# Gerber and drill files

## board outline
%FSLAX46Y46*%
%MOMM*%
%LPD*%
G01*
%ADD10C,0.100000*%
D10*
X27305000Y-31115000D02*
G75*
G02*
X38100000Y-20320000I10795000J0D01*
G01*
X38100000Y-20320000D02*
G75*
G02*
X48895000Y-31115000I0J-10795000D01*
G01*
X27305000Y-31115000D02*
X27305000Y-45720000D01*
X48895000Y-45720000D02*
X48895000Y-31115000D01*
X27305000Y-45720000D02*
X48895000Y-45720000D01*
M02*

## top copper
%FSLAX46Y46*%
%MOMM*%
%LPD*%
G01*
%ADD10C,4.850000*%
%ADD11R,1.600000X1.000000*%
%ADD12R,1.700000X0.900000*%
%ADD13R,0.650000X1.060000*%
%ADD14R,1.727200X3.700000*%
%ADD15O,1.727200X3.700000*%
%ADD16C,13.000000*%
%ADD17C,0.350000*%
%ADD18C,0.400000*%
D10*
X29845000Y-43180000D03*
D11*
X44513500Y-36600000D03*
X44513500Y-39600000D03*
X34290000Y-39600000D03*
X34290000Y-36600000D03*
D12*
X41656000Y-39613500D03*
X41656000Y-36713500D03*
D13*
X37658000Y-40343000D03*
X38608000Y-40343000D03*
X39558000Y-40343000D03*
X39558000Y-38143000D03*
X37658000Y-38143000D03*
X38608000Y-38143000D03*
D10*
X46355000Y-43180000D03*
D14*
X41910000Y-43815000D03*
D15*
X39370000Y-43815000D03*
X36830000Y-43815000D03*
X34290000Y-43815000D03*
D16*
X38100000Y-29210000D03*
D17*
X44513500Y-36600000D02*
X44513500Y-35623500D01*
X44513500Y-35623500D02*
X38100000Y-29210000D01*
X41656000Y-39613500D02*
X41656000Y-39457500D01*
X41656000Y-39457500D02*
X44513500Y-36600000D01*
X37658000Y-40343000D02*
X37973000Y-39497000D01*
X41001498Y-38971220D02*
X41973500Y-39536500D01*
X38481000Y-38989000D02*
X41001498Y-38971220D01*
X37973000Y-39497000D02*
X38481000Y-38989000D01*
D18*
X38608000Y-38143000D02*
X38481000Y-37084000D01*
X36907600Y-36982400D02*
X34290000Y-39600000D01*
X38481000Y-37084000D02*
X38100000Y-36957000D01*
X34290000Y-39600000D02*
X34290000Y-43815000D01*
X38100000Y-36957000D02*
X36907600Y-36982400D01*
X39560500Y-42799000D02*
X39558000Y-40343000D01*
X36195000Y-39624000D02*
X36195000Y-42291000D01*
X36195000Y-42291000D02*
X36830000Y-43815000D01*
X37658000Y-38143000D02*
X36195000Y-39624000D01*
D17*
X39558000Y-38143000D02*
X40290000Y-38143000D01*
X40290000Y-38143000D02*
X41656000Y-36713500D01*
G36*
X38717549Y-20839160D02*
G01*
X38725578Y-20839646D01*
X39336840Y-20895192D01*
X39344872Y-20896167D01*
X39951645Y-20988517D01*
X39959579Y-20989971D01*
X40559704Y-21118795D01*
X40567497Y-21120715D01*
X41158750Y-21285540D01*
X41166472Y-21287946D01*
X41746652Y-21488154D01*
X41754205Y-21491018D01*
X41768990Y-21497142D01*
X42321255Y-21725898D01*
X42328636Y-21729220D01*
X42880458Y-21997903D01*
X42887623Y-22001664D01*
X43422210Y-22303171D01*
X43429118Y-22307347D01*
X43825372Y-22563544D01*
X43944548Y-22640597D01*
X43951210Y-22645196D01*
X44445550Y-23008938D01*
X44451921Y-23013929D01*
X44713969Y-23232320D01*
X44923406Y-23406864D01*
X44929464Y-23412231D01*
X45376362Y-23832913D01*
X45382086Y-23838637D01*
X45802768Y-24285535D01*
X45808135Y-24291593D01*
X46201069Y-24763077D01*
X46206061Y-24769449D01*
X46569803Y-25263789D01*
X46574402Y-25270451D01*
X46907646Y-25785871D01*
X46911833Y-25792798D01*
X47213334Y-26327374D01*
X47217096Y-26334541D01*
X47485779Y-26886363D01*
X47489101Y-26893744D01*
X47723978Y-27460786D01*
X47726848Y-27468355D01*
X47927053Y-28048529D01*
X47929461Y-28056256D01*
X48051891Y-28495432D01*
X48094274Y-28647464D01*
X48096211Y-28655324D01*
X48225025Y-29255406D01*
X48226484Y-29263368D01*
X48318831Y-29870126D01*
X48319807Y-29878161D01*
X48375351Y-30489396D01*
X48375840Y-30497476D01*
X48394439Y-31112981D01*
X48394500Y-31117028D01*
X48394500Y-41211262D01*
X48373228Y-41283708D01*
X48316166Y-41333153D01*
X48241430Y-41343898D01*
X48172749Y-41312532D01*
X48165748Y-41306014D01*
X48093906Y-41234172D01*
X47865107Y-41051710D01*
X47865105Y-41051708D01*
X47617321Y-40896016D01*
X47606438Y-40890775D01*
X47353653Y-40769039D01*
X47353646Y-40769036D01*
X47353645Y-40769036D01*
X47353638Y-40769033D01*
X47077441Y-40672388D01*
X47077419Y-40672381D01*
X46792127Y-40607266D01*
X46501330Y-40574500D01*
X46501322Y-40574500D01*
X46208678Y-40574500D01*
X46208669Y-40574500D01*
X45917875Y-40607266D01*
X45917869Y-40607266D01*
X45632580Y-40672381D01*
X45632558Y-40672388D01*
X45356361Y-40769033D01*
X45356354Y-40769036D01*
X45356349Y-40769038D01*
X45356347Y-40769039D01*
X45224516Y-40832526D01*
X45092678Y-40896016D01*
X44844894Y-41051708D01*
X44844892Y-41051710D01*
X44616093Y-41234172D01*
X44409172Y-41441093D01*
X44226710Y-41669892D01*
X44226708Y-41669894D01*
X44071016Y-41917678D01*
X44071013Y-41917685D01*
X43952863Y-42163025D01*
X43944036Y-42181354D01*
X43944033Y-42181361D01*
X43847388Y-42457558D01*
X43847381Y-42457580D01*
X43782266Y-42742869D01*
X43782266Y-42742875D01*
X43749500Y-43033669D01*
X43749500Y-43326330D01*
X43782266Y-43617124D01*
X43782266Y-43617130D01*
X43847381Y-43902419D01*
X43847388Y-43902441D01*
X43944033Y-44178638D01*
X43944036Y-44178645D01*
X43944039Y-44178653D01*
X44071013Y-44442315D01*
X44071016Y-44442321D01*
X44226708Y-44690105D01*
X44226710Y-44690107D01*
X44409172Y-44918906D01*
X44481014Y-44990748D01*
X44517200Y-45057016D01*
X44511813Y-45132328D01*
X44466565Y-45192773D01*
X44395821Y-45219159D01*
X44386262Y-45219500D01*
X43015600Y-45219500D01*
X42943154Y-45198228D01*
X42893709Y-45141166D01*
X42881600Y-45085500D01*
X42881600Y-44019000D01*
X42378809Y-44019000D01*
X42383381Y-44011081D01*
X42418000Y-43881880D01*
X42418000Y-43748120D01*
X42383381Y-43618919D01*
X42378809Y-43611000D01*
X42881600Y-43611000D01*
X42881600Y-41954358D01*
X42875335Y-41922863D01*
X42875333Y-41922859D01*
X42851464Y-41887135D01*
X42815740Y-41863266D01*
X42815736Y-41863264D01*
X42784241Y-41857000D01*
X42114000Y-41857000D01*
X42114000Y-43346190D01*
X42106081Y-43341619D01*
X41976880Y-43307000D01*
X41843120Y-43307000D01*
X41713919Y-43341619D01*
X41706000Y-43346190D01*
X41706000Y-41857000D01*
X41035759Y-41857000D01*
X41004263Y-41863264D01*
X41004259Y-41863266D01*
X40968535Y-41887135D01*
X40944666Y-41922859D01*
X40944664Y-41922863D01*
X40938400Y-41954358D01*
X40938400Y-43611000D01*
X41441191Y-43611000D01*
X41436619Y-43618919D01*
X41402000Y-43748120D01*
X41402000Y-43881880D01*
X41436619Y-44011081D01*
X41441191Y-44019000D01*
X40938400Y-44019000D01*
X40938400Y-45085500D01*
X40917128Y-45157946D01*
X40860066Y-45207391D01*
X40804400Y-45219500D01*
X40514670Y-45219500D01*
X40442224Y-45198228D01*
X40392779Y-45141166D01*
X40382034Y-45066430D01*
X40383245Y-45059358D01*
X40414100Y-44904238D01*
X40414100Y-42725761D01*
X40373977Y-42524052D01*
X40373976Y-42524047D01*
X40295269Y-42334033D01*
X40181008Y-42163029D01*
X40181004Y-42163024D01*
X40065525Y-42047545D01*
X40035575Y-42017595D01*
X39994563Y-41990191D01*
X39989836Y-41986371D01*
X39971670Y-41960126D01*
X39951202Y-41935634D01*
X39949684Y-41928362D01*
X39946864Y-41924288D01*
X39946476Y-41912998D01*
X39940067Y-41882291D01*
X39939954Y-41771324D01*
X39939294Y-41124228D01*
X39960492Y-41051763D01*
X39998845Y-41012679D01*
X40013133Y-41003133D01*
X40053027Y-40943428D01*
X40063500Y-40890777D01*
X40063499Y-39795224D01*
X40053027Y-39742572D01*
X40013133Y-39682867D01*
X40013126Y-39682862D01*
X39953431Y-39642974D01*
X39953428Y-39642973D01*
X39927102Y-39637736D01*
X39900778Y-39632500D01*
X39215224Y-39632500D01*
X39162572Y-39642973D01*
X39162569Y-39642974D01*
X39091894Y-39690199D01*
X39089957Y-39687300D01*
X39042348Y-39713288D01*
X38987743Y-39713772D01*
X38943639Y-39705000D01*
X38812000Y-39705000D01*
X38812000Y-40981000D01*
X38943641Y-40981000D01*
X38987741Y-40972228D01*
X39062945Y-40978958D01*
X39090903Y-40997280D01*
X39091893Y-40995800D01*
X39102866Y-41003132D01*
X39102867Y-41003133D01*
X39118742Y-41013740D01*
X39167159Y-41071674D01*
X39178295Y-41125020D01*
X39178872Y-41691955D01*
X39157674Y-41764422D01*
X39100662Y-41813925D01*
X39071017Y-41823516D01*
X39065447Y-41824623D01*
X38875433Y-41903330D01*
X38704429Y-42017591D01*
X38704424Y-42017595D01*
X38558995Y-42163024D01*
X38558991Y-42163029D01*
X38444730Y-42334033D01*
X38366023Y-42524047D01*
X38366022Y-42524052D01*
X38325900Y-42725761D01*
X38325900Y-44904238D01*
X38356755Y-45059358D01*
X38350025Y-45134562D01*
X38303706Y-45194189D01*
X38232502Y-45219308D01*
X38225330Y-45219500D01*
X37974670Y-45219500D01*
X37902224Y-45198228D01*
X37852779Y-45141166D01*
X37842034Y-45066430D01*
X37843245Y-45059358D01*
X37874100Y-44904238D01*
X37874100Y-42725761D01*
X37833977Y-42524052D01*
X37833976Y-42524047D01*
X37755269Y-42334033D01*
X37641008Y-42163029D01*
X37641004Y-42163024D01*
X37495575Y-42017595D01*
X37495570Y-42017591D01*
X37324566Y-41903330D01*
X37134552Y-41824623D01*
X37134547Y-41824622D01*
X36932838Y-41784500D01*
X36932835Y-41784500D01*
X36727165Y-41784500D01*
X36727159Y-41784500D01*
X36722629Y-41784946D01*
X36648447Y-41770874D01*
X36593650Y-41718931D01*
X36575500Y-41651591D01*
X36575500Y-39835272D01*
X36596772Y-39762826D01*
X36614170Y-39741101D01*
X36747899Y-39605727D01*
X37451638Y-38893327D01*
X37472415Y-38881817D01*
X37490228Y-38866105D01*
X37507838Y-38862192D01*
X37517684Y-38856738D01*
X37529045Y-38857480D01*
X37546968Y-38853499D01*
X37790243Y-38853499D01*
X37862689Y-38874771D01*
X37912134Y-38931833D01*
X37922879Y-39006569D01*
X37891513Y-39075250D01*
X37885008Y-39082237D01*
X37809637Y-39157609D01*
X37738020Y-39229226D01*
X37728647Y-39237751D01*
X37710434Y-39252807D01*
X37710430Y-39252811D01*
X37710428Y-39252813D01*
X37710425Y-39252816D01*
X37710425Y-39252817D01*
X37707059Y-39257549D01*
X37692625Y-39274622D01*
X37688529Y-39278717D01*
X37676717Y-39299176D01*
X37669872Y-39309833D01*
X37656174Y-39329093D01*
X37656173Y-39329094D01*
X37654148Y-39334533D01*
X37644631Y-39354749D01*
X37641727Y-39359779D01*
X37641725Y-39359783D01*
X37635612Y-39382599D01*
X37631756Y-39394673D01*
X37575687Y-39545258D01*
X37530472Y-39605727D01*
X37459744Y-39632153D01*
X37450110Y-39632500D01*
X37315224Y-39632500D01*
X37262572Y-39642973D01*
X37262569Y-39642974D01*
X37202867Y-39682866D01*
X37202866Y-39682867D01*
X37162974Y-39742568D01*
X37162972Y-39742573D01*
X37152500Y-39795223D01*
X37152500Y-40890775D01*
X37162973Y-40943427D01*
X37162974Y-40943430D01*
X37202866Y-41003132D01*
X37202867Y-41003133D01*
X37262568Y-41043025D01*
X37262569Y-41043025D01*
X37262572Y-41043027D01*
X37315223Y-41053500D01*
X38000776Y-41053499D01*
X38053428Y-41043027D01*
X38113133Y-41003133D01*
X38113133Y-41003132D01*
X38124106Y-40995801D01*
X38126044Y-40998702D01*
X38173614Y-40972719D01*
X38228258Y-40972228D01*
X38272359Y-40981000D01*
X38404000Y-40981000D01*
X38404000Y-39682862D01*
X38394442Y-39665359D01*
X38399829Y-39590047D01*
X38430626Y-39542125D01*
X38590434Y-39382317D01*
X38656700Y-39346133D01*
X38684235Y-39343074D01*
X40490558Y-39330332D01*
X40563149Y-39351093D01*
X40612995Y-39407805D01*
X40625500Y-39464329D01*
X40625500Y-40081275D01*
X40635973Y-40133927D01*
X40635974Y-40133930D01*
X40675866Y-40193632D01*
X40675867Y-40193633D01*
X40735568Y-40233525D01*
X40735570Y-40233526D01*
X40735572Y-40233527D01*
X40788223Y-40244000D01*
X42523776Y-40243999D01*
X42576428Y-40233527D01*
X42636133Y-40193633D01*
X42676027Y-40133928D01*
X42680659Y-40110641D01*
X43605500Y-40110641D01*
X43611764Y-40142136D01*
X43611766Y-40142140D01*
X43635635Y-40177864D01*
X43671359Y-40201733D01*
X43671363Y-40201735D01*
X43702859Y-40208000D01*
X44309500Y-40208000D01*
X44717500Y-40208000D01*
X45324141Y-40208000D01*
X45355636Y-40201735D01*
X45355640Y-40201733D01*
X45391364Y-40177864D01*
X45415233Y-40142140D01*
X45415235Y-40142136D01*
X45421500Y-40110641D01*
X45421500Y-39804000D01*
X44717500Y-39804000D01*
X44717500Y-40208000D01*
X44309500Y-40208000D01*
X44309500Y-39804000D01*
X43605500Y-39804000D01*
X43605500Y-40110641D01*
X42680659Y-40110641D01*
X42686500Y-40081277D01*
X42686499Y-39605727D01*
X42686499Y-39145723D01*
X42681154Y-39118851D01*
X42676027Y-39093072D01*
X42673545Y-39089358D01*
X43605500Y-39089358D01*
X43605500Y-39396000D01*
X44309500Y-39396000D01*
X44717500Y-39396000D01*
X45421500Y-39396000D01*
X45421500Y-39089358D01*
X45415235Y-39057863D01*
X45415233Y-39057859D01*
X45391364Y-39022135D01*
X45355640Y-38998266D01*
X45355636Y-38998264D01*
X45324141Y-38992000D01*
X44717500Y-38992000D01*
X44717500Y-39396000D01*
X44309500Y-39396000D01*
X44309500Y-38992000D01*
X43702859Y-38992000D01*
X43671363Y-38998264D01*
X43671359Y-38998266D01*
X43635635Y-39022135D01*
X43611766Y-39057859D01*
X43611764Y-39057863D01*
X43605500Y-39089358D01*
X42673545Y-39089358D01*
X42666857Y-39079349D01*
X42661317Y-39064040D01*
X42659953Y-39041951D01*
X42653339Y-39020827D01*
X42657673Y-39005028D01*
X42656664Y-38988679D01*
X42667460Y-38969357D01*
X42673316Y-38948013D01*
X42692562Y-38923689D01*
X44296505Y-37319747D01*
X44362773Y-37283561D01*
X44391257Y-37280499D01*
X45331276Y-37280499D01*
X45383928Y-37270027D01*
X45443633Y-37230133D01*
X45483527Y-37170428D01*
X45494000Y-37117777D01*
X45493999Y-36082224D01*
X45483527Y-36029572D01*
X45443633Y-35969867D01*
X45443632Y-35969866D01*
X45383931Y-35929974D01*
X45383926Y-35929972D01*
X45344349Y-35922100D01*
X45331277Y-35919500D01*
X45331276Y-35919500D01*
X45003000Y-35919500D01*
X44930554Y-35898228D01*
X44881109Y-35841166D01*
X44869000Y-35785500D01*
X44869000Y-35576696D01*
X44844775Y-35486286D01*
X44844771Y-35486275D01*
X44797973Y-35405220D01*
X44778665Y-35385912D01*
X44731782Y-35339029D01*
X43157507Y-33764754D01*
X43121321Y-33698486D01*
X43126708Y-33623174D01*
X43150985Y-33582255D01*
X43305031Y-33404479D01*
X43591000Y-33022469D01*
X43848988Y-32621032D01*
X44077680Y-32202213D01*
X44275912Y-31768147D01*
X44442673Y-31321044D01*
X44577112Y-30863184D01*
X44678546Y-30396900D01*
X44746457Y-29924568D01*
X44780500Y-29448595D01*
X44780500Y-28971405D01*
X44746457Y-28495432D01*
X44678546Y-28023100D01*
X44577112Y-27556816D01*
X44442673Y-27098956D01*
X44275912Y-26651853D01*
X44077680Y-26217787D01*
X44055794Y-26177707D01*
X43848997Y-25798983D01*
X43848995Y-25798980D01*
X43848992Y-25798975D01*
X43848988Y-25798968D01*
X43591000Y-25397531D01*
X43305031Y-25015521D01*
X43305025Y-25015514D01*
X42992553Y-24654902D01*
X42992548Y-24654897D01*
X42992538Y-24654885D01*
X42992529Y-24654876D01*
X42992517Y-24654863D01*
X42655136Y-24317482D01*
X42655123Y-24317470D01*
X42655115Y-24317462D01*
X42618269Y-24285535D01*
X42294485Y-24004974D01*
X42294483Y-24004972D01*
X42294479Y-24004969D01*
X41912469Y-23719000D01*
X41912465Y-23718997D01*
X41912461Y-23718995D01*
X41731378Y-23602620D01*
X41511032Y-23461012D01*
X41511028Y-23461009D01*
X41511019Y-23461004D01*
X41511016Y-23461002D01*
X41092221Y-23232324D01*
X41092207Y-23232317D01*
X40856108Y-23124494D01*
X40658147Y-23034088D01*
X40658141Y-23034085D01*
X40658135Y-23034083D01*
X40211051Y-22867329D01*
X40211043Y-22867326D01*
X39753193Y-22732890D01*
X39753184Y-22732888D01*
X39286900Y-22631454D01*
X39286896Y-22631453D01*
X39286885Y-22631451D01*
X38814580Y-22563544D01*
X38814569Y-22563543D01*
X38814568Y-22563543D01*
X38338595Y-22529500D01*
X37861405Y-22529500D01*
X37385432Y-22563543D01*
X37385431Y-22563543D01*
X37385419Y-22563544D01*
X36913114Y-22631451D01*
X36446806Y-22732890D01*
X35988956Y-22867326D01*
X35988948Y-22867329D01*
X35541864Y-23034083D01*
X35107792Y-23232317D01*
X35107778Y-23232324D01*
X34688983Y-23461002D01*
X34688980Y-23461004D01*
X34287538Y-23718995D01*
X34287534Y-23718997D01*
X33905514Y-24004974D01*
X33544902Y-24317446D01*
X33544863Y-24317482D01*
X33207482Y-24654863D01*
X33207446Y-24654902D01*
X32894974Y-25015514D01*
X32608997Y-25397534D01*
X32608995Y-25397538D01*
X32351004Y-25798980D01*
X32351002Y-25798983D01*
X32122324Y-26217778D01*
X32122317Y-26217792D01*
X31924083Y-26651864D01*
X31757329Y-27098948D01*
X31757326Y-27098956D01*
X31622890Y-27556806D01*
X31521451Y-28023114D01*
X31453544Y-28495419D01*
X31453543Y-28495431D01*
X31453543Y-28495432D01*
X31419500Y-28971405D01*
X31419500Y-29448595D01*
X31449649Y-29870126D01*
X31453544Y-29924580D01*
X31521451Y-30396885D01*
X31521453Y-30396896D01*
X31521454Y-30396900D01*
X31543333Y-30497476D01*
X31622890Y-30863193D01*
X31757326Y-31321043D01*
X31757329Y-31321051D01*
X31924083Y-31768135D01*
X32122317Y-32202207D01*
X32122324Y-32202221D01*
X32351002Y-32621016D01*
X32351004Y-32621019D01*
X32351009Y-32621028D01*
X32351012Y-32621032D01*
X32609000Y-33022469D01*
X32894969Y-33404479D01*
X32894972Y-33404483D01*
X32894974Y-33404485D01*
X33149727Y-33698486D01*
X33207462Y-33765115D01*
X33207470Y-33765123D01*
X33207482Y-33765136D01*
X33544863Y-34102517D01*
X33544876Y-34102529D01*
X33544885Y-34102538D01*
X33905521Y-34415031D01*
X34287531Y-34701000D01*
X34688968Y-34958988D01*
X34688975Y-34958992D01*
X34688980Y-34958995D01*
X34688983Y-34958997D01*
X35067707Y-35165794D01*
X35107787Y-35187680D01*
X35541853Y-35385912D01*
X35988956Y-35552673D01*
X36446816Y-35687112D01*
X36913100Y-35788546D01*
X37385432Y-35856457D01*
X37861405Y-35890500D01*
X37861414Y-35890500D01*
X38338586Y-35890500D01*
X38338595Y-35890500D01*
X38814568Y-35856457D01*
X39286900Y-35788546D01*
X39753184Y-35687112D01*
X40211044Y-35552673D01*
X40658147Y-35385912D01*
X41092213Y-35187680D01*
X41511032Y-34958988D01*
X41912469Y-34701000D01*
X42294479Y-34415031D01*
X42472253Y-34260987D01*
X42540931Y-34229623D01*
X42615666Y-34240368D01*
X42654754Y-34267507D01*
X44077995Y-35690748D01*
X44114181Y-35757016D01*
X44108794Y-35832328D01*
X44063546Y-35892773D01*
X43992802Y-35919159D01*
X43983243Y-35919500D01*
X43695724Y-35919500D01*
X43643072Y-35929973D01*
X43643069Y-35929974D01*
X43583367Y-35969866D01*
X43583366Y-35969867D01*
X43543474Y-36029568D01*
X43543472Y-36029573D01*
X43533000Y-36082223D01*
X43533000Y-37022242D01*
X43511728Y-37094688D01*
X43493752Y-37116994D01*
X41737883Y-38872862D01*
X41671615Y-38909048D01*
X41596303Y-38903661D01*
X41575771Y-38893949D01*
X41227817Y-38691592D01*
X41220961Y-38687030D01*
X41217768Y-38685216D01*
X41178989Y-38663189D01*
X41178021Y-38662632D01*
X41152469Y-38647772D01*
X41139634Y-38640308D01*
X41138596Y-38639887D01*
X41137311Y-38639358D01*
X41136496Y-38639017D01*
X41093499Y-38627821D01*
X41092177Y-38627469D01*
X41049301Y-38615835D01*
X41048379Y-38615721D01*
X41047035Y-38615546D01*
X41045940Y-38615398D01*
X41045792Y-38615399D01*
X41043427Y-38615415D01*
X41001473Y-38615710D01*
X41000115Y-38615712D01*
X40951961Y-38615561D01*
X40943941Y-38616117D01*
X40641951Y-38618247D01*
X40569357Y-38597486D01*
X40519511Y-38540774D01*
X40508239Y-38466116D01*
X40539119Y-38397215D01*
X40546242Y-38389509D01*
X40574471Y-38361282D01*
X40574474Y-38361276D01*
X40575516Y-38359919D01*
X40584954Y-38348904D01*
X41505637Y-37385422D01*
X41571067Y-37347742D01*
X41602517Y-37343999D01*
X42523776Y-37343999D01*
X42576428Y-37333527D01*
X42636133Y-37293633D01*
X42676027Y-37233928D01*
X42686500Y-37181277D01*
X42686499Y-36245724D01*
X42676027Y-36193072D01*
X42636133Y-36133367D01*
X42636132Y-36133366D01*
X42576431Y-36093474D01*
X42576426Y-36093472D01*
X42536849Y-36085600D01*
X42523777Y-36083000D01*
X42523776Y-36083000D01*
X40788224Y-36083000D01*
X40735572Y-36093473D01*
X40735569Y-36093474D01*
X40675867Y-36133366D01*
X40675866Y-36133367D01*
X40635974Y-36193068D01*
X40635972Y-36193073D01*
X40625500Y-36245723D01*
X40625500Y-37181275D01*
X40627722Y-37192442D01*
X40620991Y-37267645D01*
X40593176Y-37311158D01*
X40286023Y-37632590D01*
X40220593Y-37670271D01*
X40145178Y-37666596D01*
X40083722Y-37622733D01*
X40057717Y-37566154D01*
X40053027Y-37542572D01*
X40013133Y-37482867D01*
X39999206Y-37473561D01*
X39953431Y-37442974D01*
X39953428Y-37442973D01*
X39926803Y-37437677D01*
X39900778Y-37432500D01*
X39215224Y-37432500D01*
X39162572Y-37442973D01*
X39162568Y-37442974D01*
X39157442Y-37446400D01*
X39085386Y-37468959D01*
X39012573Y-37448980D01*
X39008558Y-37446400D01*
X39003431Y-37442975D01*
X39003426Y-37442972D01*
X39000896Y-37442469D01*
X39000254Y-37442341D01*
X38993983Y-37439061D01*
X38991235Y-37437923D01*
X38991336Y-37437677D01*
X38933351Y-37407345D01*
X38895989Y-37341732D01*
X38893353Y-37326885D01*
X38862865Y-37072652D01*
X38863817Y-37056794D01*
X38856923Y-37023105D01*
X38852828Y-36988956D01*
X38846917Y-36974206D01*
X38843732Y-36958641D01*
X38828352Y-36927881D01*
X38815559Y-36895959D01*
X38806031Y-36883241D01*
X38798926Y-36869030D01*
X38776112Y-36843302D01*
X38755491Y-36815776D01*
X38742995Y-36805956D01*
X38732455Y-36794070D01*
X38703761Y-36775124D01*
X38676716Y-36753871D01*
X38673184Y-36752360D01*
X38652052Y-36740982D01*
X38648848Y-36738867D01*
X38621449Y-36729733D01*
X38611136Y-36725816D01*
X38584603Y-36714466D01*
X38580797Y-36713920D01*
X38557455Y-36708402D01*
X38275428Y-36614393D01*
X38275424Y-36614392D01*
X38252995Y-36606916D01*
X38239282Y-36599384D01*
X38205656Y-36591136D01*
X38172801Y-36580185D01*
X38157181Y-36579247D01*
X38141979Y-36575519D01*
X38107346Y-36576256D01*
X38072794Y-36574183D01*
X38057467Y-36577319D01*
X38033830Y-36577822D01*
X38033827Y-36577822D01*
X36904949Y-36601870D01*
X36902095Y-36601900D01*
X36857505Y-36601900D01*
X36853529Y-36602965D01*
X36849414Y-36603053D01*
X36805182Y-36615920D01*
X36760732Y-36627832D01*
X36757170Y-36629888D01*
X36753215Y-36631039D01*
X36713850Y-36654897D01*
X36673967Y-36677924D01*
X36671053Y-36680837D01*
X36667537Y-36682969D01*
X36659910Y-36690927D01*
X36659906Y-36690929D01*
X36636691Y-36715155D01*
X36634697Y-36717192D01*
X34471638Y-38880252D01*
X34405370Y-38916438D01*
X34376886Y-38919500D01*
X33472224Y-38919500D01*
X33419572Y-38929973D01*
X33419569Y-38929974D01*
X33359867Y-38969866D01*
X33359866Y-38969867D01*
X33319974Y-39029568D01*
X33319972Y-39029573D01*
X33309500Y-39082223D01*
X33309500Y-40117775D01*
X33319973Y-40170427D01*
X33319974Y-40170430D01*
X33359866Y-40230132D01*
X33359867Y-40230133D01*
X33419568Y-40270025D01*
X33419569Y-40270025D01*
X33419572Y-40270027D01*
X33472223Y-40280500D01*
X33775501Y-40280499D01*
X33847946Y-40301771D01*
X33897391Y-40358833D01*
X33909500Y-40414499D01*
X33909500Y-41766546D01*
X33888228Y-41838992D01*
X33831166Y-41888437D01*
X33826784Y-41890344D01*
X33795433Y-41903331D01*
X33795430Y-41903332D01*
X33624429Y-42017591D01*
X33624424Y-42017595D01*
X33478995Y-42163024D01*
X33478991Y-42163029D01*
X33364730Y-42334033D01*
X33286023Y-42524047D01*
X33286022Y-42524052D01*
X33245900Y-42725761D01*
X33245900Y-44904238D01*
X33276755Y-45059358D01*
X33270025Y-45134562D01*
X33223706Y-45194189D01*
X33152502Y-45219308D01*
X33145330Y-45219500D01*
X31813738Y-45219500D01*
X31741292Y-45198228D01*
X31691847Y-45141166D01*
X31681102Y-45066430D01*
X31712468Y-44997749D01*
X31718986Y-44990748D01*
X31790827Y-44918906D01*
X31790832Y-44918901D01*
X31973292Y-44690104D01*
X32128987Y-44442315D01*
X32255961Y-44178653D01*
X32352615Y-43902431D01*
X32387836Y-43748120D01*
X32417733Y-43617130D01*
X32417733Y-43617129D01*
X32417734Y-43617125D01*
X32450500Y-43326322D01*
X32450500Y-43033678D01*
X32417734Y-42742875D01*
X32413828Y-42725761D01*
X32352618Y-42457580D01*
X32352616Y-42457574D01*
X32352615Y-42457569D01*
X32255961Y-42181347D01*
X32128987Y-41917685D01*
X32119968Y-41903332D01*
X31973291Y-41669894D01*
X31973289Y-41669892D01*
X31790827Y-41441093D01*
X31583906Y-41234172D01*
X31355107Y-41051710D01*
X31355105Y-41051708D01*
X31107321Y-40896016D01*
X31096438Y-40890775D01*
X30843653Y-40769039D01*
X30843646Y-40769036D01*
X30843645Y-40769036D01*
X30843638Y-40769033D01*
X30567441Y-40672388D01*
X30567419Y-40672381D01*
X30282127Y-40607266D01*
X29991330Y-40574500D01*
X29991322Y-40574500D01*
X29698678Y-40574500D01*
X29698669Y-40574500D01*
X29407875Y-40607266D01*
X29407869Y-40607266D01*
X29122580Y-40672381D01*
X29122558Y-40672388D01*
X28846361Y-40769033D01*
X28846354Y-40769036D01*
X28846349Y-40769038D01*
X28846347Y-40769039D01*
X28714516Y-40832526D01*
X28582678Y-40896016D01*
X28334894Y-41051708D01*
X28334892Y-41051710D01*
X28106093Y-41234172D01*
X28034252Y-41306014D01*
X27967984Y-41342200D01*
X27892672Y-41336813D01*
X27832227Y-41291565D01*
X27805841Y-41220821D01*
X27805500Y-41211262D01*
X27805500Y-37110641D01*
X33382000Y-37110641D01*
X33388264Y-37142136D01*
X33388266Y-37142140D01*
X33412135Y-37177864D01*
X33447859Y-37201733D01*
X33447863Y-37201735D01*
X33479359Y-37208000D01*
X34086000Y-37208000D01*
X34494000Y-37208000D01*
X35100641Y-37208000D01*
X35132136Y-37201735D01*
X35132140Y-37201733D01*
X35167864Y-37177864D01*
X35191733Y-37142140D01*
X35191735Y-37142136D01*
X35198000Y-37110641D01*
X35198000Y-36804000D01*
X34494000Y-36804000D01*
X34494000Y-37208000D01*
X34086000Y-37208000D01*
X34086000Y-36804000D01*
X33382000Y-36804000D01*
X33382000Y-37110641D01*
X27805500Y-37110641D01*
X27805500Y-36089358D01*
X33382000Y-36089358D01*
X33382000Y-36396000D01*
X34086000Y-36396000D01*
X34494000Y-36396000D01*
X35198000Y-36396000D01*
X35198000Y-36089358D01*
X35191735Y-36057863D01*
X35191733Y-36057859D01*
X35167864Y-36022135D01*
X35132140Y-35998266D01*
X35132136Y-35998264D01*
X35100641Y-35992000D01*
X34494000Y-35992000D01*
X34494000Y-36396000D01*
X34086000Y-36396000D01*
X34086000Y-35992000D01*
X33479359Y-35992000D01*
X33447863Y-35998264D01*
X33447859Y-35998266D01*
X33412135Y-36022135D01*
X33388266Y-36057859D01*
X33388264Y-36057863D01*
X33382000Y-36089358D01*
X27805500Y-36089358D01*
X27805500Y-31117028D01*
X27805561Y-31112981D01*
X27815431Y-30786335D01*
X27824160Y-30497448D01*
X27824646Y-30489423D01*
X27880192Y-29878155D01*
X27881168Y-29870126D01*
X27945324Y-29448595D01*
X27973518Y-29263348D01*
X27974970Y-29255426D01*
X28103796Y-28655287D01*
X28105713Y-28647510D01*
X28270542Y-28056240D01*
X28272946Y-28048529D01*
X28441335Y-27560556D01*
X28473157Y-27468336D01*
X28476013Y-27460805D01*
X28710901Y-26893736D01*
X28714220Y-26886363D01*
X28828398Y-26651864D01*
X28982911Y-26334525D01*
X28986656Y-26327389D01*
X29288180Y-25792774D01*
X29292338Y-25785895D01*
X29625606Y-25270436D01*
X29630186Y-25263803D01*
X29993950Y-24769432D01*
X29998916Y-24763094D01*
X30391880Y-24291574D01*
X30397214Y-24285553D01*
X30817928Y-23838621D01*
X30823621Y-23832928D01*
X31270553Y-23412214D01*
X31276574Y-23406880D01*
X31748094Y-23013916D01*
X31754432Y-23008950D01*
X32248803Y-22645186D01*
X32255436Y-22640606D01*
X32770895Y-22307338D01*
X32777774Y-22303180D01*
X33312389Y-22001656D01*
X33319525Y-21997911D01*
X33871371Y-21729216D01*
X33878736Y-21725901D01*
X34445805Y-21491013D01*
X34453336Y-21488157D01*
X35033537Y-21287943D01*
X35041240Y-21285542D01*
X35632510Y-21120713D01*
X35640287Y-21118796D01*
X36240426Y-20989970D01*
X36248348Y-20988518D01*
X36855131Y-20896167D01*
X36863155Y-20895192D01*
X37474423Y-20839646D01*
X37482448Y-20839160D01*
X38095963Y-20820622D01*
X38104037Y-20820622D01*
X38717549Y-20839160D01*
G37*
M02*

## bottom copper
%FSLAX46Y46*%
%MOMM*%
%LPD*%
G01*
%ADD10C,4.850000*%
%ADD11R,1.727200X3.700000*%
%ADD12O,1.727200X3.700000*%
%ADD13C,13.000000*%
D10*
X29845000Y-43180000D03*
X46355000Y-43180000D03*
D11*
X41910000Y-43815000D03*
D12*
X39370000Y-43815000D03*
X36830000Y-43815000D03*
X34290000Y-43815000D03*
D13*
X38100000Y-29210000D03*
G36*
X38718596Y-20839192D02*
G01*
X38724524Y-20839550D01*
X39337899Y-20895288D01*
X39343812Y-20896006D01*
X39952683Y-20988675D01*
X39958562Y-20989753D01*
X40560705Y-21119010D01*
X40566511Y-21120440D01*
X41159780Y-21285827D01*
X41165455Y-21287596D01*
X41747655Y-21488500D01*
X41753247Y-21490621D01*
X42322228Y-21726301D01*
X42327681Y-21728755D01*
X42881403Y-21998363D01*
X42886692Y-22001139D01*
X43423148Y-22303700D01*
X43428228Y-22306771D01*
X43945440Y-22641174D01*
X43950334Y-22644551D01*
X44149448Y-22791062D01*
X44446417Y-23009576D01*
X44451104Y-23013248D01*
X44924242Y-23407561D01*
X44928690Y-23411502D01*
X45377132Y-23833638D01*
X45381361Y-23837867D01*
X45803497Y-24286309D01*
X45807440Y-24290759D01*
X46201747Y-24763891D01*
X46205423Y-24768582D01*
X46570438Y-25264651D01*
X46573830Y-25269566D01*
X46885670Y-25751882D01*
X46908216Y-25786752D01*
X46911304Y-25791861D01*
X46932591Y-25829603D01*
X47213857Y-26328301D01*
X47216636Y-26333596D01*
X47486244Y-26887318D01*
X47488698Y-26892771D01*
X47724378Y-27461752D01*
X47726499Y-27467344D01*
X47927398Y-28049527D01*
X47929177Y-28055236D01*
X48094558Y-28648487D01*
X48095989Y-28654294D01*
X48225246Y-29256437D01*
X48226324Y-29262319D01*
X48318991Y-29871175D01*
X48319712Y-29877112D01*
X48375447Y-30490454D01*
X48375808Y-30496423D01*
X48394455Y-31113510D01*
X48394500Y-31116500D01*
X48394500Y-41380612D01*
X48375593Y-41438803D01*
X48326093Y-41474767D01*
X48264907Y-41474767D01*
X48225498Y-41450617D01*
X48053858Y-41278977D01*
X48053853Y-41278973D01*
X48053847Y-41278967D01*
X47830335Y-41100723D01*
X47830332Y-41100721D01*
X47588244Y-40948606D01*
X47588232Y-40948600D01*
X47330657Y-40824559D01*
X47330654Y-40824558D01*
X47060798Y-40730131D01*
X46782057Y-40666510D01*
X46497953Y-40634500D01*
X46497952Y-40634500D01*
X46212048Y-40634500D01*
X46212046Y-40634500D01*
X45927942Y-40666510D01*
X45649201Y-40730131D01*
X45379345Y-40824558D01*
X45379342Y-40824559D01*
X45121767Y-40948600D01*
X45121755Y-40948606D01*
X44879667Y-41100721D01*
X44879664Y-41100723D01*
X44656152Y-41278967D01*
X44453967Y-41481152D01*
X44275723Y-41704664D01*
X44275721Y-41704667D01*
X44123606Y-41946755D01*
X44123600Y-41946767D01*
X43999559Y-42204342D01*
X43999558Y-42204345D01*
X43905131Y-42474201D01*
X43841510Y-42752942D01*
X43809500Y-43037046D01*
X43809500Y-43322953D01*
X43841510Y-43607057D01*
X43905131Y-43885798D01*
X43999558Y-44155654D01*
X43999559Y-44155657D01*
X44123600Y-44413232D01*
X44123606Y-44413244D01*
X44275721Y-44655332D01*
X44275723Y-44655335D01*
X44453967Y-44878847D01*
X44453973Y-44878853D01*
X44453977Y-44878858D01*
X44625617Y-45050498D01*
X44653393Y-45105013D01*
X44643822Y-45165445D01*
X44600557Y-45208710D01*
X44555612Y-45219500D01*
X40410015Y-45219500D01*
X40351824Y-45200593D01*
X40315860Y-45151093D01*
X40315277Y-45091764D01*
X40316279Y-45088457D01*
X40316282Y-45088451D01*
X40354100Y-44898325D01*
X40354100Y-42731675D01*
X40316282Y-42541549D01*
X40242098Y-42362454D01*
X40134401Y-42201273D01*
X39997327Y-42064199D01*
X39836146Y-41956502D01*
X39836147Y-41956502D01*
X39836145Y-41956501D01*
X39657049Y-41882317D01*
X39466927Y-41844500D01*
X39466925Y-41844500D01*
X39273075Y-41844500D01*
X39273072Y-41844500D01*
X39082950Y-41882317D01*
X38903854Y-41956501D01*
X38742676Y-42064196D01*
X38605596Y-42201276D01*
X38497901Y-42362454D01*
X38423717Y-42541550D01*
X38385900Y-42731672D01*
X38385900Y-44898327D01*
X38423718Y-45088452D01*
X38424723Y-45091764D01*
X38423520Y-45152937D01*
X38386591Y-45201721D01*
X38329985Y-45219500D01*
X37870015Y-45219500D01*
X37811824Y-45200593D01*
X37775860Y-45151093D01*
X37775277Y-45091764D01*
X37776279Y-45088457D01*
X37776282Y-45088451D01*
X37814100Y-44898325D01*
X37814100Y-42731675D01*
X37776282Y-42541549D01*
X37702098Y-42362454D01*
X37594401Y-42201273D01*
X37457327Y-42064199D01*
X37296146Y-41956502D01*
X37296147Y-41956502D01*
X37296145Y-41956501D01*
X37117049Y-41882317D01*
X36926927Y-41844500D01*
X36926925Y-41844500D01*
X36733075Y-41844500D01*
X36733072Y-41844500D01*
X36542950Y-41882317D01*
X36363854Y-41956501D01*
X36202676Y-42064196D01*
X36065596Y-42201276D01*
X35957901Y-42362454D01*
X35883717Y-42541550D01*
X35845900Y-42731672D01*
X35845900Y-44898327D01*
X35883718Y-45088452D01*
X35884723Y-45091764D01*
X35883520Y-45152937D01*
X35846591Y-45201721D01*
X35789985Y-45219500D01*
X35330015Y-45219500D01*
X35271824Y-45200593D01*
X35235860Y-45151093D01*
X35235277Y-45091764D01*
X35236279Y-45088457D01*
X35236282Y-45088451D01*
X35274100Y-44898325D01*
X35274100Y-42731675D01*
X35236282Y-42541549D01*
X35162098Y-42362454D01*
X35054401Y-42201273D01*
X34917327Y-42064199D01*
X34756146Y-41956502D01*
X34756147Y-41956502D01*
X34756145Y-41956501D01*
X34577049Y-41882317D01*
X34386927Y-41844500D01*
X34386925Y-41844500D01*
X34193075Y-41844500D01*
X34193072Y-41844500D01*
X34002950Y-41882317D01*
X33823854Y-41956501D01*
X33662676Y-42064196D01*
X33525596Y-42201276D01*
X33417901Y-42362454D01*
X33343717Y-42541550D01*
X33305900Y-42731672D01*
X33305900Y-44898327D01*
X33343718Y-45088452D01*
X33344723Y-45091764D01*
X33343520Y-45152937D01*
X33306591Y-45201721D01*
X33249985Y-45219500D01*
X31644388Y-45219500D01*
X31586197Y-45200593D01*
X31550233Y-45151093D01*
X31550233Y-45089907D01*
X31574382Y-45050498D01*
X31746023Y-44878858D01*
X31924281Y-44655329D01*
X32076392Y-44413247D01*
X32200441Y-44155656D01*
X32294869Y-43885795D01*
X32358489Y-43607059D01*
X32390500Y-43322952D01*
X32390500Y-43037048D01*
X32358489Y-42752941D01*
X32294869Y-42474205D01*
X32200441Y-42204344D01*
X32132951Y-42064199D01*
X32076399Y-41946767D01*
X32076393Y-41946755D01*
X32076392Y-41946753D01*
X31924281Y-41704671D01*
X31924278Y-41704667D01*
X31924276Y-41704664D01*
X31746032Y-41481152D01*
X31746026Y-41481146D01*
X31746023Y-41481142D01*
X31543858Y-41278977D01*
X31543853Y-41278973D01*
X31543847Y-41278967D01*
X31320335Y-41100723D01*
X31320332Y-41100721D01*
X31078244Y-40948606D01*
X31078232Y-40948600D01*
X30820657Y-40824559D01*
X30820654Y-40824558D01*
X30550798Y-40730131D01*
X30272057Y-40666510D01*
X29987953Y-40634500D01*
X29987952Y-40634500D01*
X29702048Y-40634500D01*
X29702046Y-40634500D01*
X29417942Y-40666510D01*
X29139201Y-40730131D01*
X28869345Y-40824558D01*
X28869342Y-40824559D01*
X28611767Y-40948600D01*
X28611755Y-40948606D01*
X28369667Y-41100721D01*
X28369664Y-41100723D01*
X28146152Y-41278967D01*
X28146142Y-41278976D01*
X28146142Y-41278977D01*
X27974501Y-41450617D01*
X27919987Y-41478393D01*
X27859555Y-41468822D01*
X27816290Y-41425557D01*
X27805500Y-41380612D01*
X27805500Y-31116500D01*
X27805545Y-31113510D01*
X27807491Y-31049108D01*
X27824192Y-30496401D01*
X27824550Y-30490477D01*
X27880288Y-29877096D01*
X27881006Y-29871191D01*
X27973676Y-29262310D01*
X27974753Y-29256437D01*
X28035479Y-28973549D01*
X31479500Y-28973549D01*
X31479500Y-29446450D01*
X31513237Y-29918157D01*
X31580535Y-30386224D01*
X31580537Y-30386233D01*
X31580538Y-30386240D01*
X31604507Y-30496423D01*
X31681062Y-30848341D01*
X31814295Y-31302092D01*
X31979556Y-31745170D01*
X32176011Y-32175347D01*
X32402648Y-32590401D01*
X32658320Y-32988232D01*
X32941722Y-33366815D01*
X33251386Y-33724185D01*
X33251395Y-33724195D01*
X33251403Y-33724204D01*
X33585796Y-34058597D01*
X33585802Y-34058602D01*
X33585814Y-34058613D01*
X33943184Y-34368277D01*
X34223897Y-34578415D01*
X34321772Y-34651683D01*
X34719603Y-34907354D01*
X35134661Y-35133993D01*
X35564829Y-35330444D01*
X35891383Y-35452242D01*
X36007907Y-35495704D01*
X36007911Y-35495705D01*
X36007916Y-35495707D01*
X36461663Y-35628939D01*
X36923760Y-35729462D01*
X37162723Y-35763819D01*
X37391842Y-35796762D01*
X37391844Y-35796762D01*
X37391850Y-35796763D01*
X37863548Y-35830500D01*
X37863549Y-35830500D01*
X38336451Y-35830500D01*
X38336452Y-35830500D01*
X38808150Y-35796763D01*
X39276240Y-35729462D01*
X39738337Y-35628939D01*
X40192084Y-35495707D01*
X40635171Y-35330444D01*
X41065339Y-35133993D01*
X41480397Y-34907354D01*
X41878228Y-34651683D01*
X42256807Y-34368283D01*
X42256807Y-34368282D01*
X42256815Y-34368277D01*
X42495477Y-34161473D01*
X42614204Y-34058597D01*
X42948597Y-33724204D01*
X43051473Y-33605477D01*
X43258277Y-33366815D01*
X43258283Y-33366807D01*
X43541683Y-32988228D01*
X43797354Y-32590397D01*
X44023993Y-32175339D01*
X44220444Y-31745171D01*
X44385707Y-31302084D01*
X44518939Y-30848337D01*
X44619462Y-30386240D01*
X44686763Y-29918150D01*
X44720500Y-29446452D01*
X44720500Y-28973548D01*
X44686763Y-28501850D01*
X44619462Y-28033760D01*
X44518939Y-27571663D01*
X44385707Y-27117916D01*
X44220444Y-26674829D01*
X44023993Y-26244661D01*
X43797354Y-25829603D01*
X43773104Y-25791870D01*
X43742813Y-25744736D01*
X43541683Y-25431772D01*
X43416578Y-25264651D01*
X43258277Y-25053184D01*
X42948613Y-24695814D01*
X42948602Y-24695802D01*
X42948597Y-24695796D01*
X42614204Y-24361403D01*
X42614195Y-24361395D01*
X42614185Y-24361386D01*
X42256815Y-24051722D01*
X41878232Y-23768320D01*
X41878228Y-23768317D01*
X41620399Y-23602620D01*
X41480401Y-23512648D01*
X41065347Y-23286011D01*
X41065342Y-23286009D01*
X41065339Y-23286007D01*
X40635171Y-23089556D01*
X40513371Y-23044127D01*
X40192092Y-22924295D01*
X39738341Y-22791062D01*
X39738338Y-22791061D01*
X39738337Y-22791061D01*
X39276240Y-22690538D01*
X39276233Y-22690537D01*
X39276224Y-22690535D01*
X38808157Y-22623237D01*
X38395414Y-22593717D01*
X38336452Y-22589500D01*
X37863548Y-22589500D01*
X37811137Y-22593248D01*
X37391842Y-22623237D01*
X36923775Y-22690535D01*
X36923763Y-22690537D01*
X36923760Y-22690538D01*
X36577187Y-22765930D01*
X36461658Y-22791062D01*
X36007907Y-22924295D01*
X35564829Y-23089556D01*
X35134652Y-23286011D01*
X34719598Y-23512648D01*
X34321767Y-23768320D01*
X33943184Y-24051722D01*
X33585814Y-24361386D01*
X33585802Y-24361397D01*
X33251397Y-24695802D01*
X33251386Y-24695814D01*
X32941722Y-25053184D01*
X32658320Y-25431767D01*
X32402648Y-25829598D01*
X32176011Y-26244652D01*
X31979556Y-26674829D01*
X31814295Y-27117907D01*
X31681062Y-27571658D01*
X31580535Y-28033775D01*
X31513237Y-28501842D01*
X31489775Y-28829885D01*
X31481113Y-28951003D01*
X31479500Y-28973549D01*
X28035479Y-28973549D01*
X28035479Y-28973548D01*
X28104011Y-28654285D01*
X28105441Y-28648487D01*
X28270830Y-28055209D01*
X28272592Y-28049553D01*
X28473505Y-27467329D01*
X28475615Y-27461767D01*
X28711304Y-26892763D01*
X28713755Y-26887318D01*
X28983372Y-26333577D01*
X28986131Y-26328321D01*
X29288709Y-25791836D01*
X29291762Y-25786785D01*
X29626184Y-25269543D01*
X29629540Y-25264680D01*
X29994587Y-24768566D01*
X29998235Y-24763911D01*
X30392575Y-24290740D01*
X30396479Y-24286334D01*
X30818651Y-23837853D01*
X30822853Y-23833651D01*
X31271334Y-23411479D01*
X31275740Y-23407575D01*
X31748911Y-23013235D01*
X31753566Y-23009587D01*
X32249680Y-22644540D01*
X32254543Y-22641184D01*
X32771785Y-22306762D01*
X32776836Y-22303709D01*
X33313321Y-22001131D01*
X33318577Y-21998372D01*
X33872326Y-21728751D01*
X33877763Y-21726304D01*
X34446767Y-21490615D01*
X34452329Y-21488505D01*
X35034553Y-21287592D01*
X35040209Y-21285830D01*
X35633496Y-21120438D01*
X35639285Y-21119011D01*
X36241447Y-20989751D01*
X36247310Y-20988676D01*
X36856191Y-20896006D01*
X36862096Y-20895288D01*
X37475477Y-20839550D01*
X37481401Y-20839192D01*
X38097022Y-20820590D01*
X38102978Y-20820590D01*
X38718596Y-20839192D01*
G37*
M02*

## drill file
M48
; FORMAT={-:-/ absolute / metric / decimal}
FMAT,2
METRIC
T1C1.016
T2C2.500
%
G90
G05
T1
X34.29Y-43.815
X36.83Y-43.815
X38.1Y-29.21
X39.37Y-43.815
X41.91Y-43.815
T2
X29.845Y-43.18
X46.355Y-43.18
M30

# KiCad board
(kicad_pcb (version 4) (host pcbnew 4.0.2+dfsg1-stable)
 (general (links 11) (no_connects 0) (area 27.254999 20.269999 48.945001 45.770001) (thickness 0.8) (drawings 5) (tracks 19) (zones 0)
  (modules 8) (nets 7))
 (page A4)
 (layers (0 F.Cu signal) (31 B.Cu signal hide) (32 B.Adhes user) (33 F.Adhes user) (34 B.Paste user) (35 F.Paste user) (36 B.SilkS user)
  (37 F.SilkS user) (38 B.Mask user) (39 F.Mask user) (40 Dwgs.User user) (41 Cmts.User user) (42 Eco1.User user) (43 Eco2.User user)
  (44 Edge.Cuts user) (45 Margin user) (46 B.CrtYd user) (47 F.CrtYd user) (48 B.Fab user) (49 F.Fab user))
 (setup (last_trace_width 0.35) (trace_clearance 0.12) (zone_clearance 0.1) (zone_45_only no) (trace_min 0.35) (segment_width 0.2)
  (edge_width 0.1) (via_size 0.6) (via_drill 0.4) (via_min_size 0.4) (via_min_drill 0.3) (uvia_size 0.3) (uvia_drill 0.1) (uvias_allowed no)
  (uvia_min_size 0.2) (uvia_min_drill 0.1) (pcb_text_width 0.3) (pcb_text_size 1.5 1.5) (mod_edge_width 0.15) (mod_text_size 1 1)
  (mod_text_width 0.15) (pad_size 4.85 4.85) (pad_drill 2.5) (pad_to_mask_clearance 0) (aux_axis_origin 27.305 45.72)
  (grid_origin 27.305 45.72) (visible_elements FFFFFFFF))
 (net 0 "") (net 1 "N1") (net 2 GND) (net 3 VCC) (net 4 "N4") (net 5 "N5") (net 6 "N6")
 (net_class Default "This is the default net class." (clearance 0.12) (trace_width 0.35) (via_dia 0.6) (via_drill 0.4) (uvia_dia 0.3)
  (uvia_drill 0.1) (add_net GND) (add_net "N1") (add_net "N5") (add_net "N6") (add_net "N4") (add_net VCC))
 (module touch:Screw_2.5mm (layer F.Cu) (at 29.845 43.18 90)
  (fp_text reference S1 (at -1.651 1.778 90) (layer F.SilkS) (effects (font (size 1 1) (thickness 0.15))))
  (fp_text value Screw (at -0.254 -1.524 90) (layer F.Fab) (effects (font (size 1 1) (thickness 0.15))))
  (pad 1 thru_hole circle (at 0 0 90) (size 4.85 4.85) (drill 2.5) (layers *.Cu *.Mask F.SilkS)))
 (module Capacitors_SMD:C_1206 (layer F.Cu) (at 44.5135 38.1 270)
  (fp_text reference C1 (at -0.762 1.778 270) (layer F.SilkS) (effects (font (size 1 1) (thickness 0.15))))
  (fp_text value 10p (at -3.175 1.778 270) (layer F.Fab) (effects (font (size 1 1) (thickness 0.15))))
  (pad 1 smd rect (at -1.5 0 270) (size 1 1.6) (layers F.Cu F.Paste F.Mask) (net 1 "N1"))
  (pad 2 smd rect (at 1.5 0 270) (size 1 1.6) (layers F.Cu F.Paste F.Mask) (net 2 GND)))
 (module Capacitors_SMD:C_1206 (layer F.Cu) (at 34.29 38.1 90)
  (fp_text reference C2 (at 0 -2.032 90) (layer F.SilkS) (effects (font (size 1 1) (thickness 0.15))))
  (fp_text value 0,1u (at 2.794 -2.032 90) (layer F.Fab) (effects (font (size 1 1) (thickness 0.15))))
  (pad 1 smd rect (at -1.5 0 90) (size 1 1.6) (layers F.Cu F.Paste F.Mask) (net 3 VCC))
  (pad 2 smd rect (at 1.5 0 90) (size 1 1.6) (layers F.Cu F.Paste F.Mask) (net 2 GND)))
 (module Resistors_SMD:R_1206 (layer F.Cu) (at 41.656 38.1635 90)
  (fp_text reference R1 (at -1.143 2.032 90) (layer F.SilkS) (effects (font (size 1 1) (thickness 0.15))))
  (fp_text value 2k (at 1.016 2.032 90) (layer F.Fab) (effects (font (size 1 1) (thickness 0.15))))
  (pad 1 smd rect (at -1.45 0 90) (size 0.9 1.7) (layers F.Cu F.Paste F.Mask) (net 1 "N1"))
  (pad 2 smd rect (at 1.45 0 90) (size 0.9 1.7) (layers F.Cu F.Paste F.Mask) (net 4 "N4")))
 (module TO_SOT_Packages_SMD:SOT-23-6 (layer F.Cu) (at 38.608 39.243 90)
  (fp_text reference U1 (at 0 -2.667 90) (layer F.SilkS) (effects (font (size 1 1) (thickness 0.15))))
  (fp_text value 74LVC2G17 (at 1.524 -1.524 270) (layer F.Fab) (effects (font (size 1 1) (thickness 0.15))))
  (pad 1 smd rect (at -1.1 -0.95 90) (size 1.06 0.65) (layers F.Cu F.Paste F.Mask) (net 1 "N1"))
  (pad 2 smd rect (at -1.1 0 90) (size 1.06 0.65) (layers F.Cu F.Paste F.Mask) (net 2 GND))
  (pad 3 smd rect (at -1.1 0.95 90) (size 1.06 0.65) (layers F.Cu F.Paste F.Mask) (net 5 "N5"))
  (pad 4 smd rect (at 1.1 0.95 90) (size 1.06 0.65) (layers F.Cu F.Paste F.Mask) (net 4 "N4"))
  (pad 6 smd rect (at 1.1 -0.95 90) (size 1.06 0.65) (layers F.Cu F.Paste F.Mask) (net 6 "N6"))
  (pad 5 smd rect (at 1.1 0 90) (size 1.06 0.65) (layers F.Cu F.Paste F.Mask) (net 3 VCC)))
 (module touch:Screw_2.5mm (layer F.Cu) (at 46.355 43.18 90)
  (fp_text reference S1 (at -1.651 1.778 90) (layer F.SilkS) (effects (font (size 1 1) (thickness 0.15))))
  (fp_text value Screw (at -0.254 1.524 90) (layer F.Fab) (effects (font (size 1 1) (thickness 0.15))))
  (pad 1 thru_hole circle (at 0 0 90) (size 4.85 4.85) (drill 2.5) (layers *.Cu *.Mask F.SilkS)))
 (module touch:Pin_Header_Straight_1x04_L (layer F.Cu) (at 41.91 43.815 270)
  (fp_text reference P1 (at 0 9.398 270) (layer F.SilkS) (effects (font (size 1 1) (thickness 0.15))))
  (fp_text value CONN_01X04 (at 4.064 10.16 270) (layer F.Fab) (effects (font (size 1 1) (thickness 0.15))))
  (pad 1 thru_hole rect (at 0 0 270) (size 3.7 1.7272) (drill 1.016) (layers *.Cu *.Mask F.SilkS) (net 2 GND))
  (pad 2 thru_hole oval (at 0 2.54 270) (size 3.7 1.7272) (drill 1.016) (layers *.Cu *.Mask F.SilkS) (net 5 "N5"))
  (pad 3 thru_hole oval (at 0 5.08 270) (size 3.7 1.7272) (drill 1.016) (layers *.Cu *.Mask F.SilkS) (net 6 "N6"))
  (pad 4 thru_hole oval (at 0 7.62 270) (size 3.7 1.7272) (drill 1.016) (layers *.Cu *.Mask F.SilkS) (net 3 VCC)))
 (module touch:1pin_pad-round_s (layer F.Cu) (at 38.1 29.21 90)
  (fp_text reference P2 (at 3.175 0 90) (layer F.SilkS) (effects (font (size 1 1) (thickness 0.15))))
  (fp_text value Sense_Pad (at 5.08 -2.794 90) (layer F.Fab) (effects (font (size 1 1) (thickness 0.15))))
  (pad 1 thru_hole circle (at 0 0 90) (size 13 13) (drill 1.016) (layers *.Cu *.Mask F.SilkS) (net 1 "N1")))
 (gr_arc (start 38.1 31.115) (end 27.305 31.115) (angle 90) (layer Edge.Cuts) (width 0.1))
 (gr_arc (start 38.1 31.115) (end 38.1 20.32) (angle 90) (layer Edge.Cuts) (width 0.1))
 (gr_line (start 27.305 31.115) (end 27.305 45.72) (angle 90) (layer Edge.Cuts) (width 0.1))
 (gr_line (start 48.895 45.72) (end 48.895 31.115) (angle 90) (layer Edge.Cuts) (width 0.1))
 (gr_line (start 27.305 45.72) (end 48.895 45.72) (angle 90) (layer Edge.Cuts) (width 0.1))
 (segment (start 44.5135 36.6) (end 44.5135 35.6235) (width 0.35) (layer F.Cu) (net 1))
 (segment (start 44.5135 35.6235) (end 38.1 29.21) (width 0.35) (layer F.Cu) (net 1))
 (segment (start 41.656 39.6135) (end 41.656 39.4575) (width 0.35) (layer F.Cu) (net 1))
 (segment (start 41.656 39.4575) (end 44.5135 36.6) (width 0.35) (layer F.Cu) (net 1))
 (segment (start 37.658 40.343) (end 37.973 39.497) (width 0.35) (layer F.Cu) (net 1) (status 10))
 (segment (start 41.001498 38.97122) (end 41.9735 39.5365) (width 0.35) (layer F.Cu) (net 1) (status 20))
 (segment (start 38.481 38.989) (end 41.001498 38.97122) (width 0.35) (layer F.Cu) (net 1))
 (segment (start 37.973 39.497) (end 38.481 38.989) (width 0.35) (layer F.Cu) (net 1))
 (segment (start 38.608 38.143) (end 38.481 37.084) (width 0.4) (layer F.Cu) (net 3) (status 10))
 (segment (start 36.9076 36.9824) (end 34.29 39.6) (width 0.4) (layer F.Cu) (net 3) (status 20))
 (segment (start 38.481 37.084) (end 38.1 36.957) (width 0.4) (layer F.Cu) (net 3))
 (segment (start 34.29 39.6) (end 34.29 43.815) (width 0.4) (layer F.Cu) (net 3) (status 10))
 (segment (start 38.1 36.957) (end 36.9076 36.9824) (width 0.4) (layer F.Cu) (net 3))
 (segment (start 39.5605 42.799) (end 39.558 40.343) (width 0.4) (layer F.Cu) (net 5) (status 20))
 (segment (start 36.195 39.624) (end 36.195 42.291) (width 0.4) (layer F.Cu) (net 6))
 (segment (start 36.195 42.291) (end 36.83 43.815) (width 0.4) (layer F.Cu) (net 6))
 (segment (start 37.658 38.143) (end 36.195 39.624) (width 0.4) (layer F.Cu) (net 6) (status 10))
 (segment (start 39.558 38.143) (end 40.29 38.143) (width 0.35) (layer F.Cu) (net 4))
 (segment (start 40.29 38.143) (end 41.656 36.7135) (width 0.35) (layer F.Cu) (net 4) (status 20))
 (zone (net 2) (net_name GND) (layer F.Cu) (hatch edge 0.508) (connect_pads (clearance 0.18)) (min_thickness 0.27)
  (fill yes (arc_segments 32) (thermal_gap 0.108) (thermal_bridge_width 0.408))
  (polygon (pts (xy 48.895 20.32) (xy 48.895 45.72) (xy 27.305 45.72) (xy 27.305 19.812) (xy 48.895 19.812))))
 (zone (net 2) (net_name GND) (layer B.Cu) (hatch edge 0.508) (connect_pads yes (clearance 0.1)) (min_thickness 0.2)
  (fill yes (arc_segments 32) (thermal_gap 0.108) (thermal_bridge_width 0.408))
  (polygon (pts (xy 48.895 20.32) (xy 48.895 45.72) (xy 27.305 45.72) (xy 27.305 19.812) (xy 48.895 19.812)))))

